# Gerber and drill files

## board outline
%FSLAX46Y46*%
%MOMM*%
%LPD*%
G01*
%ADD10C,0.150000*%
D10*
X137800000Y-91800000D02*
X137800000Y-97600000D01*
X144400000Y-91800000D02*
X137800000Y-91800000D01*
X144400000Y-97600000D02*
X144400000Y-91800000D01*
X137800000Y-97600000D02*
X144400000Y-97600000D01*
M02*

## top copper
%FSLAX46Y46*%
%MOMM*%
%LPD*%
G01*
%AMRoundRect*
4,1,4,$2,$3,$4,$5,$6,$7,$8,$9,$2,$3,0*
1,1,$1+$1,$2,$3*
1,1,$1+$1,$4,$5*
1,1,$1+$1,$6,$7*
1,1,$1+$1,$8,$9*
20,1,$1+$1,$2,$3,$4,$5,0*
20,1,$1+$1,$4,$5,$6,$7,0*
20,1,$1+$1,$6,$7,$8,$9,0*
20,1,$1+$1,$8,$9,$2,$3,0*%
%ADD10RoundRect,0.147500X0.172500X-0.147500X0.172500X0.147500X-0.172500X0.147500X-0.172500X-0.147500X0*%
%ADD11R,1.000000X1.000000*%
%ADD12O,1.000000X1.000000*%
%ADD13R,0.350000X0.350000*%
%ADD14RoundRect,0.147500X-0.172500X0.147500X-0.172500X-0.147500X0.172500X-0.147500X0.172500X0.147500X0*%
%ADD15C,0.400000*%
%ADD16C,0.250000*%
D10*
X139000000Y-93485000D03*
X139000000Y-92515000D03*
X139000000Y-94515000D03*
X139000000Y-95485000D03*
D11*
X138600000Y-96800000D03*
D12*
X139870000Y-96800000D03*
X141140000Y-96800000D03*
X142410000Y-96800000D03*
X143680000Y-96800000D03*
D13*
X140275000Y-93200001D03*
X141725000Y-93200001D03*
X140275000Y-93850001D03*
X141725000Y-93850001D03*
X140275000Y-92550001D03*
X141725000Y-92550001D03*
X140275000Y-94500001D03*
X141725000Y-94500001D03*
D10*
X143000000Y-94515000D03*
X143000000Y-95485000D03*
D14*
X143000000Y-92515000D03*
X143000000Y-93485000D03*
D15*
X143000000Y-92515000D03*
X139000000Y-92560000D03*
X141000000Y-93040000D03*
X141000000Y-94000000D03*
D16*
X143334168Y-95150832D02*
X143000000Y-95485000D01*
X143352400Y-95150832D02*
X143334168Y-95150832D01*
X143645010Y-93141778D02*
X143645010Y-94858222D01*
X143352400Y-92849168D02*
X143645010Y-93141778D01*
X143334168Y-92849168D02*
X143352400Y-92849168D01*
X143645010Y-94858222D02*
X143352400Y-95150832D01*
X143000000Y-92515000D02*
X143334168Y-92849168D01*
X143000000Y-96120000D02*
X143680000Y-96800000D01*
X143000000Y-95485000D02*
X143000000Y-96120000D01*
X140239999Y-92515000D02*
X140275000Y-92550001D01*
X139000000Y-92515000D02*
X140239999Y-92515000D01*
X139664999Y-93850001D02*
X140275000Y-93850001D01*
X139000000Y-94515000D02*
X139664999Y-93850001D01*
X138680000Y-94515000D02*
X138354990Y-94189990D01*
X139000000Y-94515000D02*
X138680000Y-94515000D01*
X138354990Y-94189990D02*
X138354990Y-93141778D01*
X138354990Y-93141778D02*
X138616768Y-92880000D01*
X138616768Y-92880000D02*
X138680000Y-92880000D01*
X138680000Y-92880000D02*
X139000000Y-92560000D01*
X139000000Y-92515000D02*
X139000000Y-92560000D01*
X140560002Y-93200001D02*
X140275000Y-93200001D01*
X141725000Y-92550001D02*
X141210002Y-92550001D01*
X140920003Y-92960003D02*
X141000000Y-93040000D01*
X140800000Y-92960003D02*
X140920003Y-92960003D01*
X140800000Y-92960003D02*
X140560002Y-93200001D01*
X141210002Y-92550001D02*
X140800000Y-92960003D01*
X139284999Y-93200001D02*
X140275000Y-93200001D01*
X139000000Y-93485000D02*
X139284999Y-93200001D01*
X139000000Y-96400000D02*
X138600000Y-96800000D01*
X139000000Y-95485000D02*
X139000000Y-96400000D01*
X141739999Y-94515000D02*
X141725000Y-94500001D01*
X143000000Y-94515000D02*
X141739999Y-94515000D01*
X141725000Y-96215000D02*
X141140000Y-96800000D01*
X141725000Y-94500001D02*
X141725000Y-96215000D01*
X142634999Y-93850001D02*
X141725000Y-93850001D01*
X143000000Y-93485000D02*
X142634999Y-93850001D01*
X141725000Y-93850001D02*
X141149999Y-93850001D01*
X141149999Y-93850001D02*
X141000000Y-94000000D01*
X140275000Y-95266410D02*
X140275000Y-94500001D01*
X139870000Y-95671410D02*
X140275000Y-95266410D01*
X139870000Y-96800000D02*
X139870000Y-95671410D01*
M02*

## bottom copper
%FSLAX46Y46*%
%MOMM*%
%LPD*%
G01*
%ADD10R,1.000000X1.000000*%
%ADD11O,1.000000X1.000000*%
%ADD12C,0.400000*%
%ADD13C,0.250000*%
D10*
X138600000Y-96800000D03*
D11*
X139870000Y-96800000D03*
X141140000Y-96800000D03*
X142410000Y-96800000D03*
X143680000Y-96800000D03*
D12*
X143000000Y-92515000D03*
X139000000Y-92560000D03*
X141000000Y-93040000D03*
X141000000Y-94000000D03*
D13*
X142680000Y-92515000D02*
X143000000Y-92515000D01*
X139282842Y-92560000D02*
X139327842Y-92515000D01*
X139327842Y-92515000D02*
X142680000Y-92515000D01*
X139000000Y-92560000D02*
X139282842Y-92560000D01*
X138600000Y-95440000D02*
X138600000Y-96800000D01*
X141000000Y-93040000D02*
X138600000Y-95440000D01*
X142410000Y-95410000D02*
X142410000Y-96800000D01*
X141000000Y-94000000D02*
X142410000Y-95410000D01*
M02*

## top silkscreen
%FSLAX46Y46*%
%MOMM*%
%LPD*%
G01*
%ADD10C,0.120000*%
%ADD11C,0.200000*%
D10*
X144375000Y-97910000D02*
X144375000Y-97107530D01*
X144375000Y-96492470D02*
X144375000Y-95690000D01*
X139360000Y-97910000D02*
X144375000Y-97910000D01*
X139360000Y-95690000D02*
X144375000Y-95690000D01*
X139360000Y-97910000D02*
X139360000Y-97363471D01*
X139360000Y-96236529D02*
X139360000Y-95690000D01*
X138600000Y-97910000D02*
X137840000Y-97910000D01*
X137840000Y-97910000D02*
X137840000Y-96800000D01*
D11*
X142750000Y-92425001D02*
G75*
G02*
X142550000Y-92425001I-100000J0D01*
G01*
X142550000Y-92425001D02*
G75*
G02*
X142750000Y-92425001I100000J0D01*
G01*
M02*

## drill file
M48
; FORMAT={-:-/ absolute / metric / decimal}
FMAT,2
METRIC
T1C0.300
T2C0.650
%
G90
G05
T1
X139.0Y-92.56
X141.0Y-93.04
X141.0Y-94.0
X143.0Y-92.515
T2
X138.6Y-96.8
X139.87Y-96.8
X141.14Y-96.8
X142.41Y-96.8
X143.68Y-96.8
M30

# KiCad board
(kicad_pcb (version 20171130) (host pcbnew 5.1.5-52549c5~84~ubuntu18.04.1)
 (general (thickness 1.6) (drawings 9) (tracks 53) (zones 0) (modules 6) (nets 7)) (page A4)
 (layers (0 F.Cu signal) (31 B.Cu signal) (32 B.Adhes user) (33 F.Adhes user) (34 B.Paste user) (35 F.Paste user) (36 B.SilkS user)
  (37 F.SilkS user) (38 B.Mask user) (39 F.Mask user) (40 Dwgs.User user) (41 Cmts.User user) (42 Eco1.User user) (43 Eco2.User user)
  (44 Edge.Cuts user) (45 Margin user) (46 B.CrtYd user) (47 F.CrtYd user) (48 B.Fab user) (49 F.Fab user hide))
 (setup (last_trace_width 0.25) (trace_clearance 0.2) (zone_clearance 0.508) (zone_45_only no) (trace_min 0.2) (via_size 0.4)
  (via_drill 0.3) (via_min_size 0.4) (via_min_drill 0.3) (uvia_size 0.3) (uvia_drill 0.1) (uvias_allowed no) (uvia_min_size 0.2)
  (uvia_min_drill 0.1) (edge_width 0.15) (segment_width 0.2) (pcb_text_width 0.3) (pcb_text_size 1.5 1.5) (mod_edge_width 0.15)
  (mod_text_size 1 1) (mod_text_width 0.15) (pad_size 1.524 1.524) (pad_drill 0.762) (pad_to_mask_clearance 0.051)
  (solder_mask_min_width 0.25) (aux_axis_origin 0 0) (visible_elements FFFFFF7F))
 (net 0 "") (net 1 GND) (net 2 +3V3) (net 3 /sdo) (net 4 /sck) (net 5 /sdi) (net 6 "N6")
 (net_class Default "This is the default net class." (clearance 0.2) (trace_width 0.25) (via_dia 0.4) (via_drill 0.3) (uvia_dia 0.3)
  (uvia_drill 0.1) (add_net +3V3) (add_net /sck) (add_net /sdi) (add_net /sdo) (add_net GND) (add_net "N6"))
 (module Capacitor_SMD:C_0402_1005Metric (layer F.Cu) (at 139 93 90)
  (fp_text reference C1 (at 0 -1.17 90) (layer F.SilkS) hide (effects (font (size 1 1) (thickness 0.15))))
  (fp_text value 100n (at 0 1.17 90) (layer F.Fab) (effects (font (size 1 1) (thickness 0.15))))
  (pad 1 smd roundrect (at -0.485 0 90) (size 0.59 0.64) (layers F.Cu F.Paste F.Mask) (roundrect_rratio 0.25) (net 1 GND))
  (pad 2 smd roundrect (at 0.485 0 90) (size 0.59 0.64) (layers F.Cu F.Paste F.Mask) (roundrect_rratio 0.25) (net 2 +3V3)))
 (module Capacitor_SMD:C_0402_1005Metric (layer F.Cu) (at 139 95 90)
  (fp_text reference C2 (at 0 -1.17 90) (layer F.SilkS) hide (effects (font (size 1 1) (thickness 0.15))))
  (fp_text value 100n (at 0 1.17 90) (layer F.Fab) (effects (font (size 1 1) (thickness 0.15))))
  (pad 2 smd roundrect (at 0.485 0 90) (size 0.59 0.64) (layers F.Cu F.Paste F.Mask) (roundrect_rratio 0.25) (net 2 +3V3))
  (pad 1 smd roundrect (at -0.485 0 90) (size 0.59 0.64) (layers F.Cu F.Paste F.Mask) (roundrect_rratio 0.25) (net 1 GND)))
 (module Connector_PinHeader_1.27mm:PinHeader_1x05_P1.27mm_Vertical (layer F.Cu) (at 138.6 96.8 90)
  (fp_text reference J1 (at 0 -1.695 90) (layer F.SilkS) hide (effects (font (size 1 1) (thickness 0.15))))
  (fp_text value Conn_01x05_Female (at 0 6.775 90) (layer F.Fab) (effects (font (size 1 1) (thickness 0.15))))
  (fp_line (start -1.11 5.775) (end -0.30753 5.775) (layer F.SilkS) (width 0.12))
  (fp_line (start 0.30753 5.775) (end 1.11 5.775) (layer F.SilkS) (width 0.12))
  (fp_line (start -1.11 0.76) (end -1.11 5.775) (layer F.SilkS) (width 0.12))
  (fp_line (start 1.11 0.76) (end 1.11 5.775) (layer F.SilkS) (width 0.12))
  (fp_line (start -1.11 0.76) (end -0.563471 0.76) (layer F.SilkS) (width 0.12))
  (fp_line (start 0.563471 0.76) (end 1.11 0.76) (layer F.SilkS) (width 0.12))
  (fp_line (start -1.11 0) (end -1.11 -0.76) (layer F.SilkS) (width 0.12))
  (fp_line (start -1.11 -0.76) (end 0 -0.76) (layer F.SilkS) (width 0.12))
  (pad 1 thru_hole rect (at 0 0 90) (size 1 1) (drill 0.65) (layers *.Cu *.Mask) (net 1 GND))
  (pad 2 thru_hole oval (at 0 1.27 90) (size 1 1) (drill 0.65) (layers *.Cu *.Mask) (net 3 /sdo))
  (pad 3 thru_hole oval (at 0 2.54 90) (size 1 1) (drill 0.65) (layers *.Cu *.Mask) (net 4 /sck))
  (pad 4 thru_hole oval (at 0 3.81 90) (size 1 1) (drill 0.65) (layers *.Cu *.Mask) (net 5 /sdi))
  (pad 5 thru_hole oval (at 0 5.08 90) (size 1 1) (drill 0.65) (layers *.Cu *.Mask) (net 2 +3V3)))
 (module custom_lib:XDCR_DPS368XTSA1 (layer F.Cu) (at 141 93.525001)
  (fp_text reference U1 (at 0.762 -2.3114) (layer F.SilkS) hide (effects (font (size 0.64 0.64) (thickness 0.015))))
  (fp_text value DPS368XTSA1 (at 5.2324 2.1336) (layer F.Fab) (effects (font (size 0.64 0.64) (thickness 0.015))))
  (fp_circle (center 1.65 -1.1) (end 1.75 -1.1) (layer F.SilkS) (width 0.2))
  (pad 7 smd rect (at -0.725 -0.325) (size 0.35 0.35) (layers F.Cu F.Mask) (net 1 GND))
  (pad 2 smd rect (at 0.725 -0.325) (size 0.35 0.35) (layers F.Cu F.Mask) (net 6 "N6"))
  (pad 6 smd rect (at -0.725 0.325) (size 0.35 0.35) (layers F.Cu F.Mask) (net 2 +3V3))
  (pad 3 smd rect (at 0.725 0.325) (size 0.35 0.35) (layers F.Cu F.Mask) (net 5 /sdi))
  (pad 8 smd rect (at -0.725 -0.975) (size 0.35 0.35) (layers F.Cu F.Mask) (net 2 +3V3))
  (pad 1 smd rect (at 0.725 -0.975) (size 0.35 0.35) (layers F.Cu F.Mask) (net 1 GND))
  (pad 5 smd rect (at -0.725 0.975) (size 0.35 0.35) (layers F.Cu F.Mask) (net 3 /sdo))
  (pad 4 smd rect (at 0.725 0.975) (size 0.35 0.35) (layers F.Cu F.Mask) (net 4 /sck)))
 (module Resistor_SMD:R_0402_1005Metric (layer F.Cu) (at 143 95 90)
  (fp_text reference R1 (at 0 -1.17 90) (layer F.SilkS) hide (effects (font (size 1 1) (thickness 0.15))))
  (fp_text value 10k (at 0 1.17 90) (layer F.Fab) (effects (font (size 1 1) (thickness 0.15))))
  (pad 2 smd roundrect (at 0.485 0 90) (size 0.59 0.64) (layers F.Cu F.Paste F.Mask) (roundrect_rratio 0.25) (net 4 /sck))
  (pad 1 smd roundrect (at -0.485 0 90) (size 0.59 0.64) (layers F.Cu F.Paste F.Mask) (roundrect_rratio 0.25) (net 2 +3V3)))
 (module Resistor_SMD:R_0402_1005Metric (layer F.Cu) (at 143 93 270)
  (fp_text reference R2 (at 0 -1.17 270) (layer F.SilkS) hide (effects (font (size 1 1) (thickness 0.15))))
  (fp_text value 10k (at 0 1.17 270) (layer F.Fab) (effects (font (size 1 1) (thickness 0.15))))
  (pad 1 smd roundrect (at -0.485 0 270) (size 0.59 0.64) (layers F.Cu F.Paste F.Mask) (roundrect_rratio 0.25) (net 2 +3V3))
  (pad 2 smd roundrect (at 0.485 0 270) (size 0.59 0.64) (layers F.Cu F.Paste F.Mask) (roundrect_rratio 0.25) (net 5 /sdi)))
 (gr_line (start 137.8 91.8) (end 137.8 97.6) (layer Edge.Cuts) (width 0.15))
 (gr_line (start 144.4 91.8) (end 137.8 91.8) (layer Edge.Cuts) (width 0.15))
 (gr_line (start 144.4 97.6) (end 144.4 91.8) (layer Edge.Cuts) (width 0.15))
 (gr_line (start 137.8 97.6) (end 144.4 97.6) (layer Edge.Cuts) (width 0.15))
 (segment (start 143.334168 95.150832) (end 143 95.485) (width 0.25) (layer F.Cu) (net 2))
 (segment (start 143.3524 95.150832) (end 143.334168 95.150832) (width 0.25) (layer F.Cu) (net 2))
 (segment (start 143.64501 93.141778) (end 143.64501 94.858222) (width 0.25) (layer F.Cu) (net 2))
 (segment (start 143.3524 92.849168) (end 143.64501 93.141778) (width 0.25) (layer F.Cu) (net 2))
 (segment (start 143.334168 92.849168) (end 143.3524 92.849168) (width 0.25) (layer F.Cu) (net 2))
 (segment (start 143.64501 94.858222) (end 143.3524 95.150832) (width 0.25) (layer F.Cu) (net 2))
 (segment (start 143 92.515) (end 143.334168 92.849168) (width 0.25) (layer F.Cu) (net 2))
 (segment (start 143 96.12) (end 143.68 96.8) (width 0.25) (layer F.Cu) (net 2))
 (segment (start 143 95.485) (end 143 96.12) (width 0.25) (layer F.Cu) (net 2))
 (via (at 143 92.515) (size 0.4) (drill 0.3) (layers F.Cu B.Cu) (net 2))
 (segment (start 140.239999 92.515) (end 140.275 92.550001) (width 0.25) (layer F.Cu) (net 2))
 (segment (start 139 92.515) (end 140.239999 92.515) (width 0.25) (layer F.Cu) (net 2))
 (segment (start 139.664999 93.850001) (end 140.275 93.850001) (width 0.25) (layer F.Cu) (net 2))
 (segment (start 139 94.515) (end 139.664999 93.850001) (width 0.25) (layer F.Cu) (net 2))
 (segment (start 138.68 94.515) (end 138.35499 94.18999) (width 0.25) (layer F.Cu) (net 2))
 (segment (start 139 94.515) (end 138.68 94.515) (width 0.25) (layer F.Cu) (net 2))
 (segment (start 138.35499 94.18999) (end 138.35499 93.141778) (width 0.25) (layer F.Cu) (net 2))
 (segment (start 138.35499 93.141778) (end 138.616768 92.88) (width 0.25) (layer F.Cu) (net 2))
 (segment (start 138.616768 92.88) (end 138.68 92.88) (width 0.25) (layer F.Cu) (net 2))
 (segment (start 138.68 92.88) (end 139 92.56) (width 0.25) (layer F.Cu) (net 2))
 (via (at 139 92.56) (size 0.4) (drill 0.3) (layers F.Cu B.Cu) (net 2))
 (segment (start 139 92.515) (end 139 92.56) (width 0.25) (layer F.Cu) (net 2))
 (segment (start 142.68 92.515) (end 143 92.515) (width 0.25) (layer B.Cu) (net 2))
 (segment (start 139.282842 92.56) (end 139.327842 92.515) (width 0.25) (layer B.Cu) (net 2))
 (segment (start 139.327842 92.515) (end 142.68 92.515) (width 0.25) (layer B.Cu) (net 2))
 (segment (start 139 92.56) (end 139.282842 92.56) (width 0.25) (layer B.Cu) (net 2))
 (segment (start 140.560002 93.200001) (end 140.275 93.200001) (width 0.25) (layer F.Cu) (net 1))
 (segment (start 141.725 92.550001) (end 141.210002 92.550001) (width 0.25) (layer F.Cu) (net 1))
 (via (at 141 93.04) (size 0.4) (drill 0.3) (layers F.Cu B.Cu) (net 1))
 (segment (start 140.920003 92.960003) (end 141 93.04) (width 0.25) (layer F.Cu) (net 1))
 (segment (start 140.8 92.960003) (end 140.920003 92.960003) (width 0.25) (layer F.Cu) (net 1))
 (segment (start 140.8 92.960003) (end 140.560002 93.200001) (width 0.25) (layer F.Cu) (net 1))
 (segment (start 141.210002 92.550001) (end 140.8 92.960003) (width 0.25) (layer F.Cu) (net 1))
 (segment (start 138.6 95.44) (end 138.6 96.8) (width 0.25) (layer B.Cu) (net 1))
 (segment (start 141 93.04) (end 138.6 95.44) (width 0.25) (layer B.Cu) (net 1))
 (segment (start 139.284999 93.200001) (end 140.275 93.200001) (width 0.25) (layer F.Cu) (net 1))
 (segment (start 139 93.485) (end 139.284999 93.200001) (width 0.25) (layer F.Cu) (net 1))
 (segment (start 139 96.4) (end 138.6 96.8) (width 0.25) (layer F.Cu) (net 1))
 (segment (start 139 95.485) (end 139 96.4) (width 0.25) (layer F.Cu) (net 1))
 (segment (start 141.739999 94.515) (end 141.725 94.500001) (width 0.25) (layer F.Cu) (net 4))
 (segment (start 143 94.515) (end 141.739999 94.515) (width 0.25) (layer F.Cu) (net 4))
 (segment (start 141.725 96.215) (end 141.14 96.8) (width 0.25) (layer F.Cu) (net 4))
 (segment (start 141.725 94.500001) (end 141.725 96.215) (width 0.25) (layer F.Cu) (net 4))
 (segment (start 142.634999 93.850001) (end 141.725 93.850001) (width 0.25) (layer F.Cu) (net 5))
 (segment (start 143 93.485) (end 142.634999 93.850001) (width 0.25) (layer F.Cu) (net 5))
 (via (at 141 94) (size 0.4) (drill 0.3) (layers F.Cu B.Cu) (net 5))
 (segment (start 141.725 93.850001) (end 141.149999 93.850001) (width 0.25) (layer F.Cu) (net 5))
 (segment (start 141.149999 93.850001) (end 141 94) (width 0.25) (layer F.Cu) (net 5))
 (segment (start 142.41 95.41) (end 142.41 96.8) (width 0.25) (layer B.Cu) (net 5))
 (segment (start 141 94) (end 142.41 95.41) (width 0.25) (layer B.Cu) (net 5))
 (segment (start 140.275 95.26641) (end 140.275 94.500001) (width 0.25) (layer F.Cu) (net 3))
 (segment (start 139.87 95.67141) (end 140.275 95.26641) (width 0.25) (layer F.Cu) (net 3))
 (segment (start 139.87 96.8) (end 139.87 95.67141) (width 0.25) (layer F.Cu) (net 3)))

